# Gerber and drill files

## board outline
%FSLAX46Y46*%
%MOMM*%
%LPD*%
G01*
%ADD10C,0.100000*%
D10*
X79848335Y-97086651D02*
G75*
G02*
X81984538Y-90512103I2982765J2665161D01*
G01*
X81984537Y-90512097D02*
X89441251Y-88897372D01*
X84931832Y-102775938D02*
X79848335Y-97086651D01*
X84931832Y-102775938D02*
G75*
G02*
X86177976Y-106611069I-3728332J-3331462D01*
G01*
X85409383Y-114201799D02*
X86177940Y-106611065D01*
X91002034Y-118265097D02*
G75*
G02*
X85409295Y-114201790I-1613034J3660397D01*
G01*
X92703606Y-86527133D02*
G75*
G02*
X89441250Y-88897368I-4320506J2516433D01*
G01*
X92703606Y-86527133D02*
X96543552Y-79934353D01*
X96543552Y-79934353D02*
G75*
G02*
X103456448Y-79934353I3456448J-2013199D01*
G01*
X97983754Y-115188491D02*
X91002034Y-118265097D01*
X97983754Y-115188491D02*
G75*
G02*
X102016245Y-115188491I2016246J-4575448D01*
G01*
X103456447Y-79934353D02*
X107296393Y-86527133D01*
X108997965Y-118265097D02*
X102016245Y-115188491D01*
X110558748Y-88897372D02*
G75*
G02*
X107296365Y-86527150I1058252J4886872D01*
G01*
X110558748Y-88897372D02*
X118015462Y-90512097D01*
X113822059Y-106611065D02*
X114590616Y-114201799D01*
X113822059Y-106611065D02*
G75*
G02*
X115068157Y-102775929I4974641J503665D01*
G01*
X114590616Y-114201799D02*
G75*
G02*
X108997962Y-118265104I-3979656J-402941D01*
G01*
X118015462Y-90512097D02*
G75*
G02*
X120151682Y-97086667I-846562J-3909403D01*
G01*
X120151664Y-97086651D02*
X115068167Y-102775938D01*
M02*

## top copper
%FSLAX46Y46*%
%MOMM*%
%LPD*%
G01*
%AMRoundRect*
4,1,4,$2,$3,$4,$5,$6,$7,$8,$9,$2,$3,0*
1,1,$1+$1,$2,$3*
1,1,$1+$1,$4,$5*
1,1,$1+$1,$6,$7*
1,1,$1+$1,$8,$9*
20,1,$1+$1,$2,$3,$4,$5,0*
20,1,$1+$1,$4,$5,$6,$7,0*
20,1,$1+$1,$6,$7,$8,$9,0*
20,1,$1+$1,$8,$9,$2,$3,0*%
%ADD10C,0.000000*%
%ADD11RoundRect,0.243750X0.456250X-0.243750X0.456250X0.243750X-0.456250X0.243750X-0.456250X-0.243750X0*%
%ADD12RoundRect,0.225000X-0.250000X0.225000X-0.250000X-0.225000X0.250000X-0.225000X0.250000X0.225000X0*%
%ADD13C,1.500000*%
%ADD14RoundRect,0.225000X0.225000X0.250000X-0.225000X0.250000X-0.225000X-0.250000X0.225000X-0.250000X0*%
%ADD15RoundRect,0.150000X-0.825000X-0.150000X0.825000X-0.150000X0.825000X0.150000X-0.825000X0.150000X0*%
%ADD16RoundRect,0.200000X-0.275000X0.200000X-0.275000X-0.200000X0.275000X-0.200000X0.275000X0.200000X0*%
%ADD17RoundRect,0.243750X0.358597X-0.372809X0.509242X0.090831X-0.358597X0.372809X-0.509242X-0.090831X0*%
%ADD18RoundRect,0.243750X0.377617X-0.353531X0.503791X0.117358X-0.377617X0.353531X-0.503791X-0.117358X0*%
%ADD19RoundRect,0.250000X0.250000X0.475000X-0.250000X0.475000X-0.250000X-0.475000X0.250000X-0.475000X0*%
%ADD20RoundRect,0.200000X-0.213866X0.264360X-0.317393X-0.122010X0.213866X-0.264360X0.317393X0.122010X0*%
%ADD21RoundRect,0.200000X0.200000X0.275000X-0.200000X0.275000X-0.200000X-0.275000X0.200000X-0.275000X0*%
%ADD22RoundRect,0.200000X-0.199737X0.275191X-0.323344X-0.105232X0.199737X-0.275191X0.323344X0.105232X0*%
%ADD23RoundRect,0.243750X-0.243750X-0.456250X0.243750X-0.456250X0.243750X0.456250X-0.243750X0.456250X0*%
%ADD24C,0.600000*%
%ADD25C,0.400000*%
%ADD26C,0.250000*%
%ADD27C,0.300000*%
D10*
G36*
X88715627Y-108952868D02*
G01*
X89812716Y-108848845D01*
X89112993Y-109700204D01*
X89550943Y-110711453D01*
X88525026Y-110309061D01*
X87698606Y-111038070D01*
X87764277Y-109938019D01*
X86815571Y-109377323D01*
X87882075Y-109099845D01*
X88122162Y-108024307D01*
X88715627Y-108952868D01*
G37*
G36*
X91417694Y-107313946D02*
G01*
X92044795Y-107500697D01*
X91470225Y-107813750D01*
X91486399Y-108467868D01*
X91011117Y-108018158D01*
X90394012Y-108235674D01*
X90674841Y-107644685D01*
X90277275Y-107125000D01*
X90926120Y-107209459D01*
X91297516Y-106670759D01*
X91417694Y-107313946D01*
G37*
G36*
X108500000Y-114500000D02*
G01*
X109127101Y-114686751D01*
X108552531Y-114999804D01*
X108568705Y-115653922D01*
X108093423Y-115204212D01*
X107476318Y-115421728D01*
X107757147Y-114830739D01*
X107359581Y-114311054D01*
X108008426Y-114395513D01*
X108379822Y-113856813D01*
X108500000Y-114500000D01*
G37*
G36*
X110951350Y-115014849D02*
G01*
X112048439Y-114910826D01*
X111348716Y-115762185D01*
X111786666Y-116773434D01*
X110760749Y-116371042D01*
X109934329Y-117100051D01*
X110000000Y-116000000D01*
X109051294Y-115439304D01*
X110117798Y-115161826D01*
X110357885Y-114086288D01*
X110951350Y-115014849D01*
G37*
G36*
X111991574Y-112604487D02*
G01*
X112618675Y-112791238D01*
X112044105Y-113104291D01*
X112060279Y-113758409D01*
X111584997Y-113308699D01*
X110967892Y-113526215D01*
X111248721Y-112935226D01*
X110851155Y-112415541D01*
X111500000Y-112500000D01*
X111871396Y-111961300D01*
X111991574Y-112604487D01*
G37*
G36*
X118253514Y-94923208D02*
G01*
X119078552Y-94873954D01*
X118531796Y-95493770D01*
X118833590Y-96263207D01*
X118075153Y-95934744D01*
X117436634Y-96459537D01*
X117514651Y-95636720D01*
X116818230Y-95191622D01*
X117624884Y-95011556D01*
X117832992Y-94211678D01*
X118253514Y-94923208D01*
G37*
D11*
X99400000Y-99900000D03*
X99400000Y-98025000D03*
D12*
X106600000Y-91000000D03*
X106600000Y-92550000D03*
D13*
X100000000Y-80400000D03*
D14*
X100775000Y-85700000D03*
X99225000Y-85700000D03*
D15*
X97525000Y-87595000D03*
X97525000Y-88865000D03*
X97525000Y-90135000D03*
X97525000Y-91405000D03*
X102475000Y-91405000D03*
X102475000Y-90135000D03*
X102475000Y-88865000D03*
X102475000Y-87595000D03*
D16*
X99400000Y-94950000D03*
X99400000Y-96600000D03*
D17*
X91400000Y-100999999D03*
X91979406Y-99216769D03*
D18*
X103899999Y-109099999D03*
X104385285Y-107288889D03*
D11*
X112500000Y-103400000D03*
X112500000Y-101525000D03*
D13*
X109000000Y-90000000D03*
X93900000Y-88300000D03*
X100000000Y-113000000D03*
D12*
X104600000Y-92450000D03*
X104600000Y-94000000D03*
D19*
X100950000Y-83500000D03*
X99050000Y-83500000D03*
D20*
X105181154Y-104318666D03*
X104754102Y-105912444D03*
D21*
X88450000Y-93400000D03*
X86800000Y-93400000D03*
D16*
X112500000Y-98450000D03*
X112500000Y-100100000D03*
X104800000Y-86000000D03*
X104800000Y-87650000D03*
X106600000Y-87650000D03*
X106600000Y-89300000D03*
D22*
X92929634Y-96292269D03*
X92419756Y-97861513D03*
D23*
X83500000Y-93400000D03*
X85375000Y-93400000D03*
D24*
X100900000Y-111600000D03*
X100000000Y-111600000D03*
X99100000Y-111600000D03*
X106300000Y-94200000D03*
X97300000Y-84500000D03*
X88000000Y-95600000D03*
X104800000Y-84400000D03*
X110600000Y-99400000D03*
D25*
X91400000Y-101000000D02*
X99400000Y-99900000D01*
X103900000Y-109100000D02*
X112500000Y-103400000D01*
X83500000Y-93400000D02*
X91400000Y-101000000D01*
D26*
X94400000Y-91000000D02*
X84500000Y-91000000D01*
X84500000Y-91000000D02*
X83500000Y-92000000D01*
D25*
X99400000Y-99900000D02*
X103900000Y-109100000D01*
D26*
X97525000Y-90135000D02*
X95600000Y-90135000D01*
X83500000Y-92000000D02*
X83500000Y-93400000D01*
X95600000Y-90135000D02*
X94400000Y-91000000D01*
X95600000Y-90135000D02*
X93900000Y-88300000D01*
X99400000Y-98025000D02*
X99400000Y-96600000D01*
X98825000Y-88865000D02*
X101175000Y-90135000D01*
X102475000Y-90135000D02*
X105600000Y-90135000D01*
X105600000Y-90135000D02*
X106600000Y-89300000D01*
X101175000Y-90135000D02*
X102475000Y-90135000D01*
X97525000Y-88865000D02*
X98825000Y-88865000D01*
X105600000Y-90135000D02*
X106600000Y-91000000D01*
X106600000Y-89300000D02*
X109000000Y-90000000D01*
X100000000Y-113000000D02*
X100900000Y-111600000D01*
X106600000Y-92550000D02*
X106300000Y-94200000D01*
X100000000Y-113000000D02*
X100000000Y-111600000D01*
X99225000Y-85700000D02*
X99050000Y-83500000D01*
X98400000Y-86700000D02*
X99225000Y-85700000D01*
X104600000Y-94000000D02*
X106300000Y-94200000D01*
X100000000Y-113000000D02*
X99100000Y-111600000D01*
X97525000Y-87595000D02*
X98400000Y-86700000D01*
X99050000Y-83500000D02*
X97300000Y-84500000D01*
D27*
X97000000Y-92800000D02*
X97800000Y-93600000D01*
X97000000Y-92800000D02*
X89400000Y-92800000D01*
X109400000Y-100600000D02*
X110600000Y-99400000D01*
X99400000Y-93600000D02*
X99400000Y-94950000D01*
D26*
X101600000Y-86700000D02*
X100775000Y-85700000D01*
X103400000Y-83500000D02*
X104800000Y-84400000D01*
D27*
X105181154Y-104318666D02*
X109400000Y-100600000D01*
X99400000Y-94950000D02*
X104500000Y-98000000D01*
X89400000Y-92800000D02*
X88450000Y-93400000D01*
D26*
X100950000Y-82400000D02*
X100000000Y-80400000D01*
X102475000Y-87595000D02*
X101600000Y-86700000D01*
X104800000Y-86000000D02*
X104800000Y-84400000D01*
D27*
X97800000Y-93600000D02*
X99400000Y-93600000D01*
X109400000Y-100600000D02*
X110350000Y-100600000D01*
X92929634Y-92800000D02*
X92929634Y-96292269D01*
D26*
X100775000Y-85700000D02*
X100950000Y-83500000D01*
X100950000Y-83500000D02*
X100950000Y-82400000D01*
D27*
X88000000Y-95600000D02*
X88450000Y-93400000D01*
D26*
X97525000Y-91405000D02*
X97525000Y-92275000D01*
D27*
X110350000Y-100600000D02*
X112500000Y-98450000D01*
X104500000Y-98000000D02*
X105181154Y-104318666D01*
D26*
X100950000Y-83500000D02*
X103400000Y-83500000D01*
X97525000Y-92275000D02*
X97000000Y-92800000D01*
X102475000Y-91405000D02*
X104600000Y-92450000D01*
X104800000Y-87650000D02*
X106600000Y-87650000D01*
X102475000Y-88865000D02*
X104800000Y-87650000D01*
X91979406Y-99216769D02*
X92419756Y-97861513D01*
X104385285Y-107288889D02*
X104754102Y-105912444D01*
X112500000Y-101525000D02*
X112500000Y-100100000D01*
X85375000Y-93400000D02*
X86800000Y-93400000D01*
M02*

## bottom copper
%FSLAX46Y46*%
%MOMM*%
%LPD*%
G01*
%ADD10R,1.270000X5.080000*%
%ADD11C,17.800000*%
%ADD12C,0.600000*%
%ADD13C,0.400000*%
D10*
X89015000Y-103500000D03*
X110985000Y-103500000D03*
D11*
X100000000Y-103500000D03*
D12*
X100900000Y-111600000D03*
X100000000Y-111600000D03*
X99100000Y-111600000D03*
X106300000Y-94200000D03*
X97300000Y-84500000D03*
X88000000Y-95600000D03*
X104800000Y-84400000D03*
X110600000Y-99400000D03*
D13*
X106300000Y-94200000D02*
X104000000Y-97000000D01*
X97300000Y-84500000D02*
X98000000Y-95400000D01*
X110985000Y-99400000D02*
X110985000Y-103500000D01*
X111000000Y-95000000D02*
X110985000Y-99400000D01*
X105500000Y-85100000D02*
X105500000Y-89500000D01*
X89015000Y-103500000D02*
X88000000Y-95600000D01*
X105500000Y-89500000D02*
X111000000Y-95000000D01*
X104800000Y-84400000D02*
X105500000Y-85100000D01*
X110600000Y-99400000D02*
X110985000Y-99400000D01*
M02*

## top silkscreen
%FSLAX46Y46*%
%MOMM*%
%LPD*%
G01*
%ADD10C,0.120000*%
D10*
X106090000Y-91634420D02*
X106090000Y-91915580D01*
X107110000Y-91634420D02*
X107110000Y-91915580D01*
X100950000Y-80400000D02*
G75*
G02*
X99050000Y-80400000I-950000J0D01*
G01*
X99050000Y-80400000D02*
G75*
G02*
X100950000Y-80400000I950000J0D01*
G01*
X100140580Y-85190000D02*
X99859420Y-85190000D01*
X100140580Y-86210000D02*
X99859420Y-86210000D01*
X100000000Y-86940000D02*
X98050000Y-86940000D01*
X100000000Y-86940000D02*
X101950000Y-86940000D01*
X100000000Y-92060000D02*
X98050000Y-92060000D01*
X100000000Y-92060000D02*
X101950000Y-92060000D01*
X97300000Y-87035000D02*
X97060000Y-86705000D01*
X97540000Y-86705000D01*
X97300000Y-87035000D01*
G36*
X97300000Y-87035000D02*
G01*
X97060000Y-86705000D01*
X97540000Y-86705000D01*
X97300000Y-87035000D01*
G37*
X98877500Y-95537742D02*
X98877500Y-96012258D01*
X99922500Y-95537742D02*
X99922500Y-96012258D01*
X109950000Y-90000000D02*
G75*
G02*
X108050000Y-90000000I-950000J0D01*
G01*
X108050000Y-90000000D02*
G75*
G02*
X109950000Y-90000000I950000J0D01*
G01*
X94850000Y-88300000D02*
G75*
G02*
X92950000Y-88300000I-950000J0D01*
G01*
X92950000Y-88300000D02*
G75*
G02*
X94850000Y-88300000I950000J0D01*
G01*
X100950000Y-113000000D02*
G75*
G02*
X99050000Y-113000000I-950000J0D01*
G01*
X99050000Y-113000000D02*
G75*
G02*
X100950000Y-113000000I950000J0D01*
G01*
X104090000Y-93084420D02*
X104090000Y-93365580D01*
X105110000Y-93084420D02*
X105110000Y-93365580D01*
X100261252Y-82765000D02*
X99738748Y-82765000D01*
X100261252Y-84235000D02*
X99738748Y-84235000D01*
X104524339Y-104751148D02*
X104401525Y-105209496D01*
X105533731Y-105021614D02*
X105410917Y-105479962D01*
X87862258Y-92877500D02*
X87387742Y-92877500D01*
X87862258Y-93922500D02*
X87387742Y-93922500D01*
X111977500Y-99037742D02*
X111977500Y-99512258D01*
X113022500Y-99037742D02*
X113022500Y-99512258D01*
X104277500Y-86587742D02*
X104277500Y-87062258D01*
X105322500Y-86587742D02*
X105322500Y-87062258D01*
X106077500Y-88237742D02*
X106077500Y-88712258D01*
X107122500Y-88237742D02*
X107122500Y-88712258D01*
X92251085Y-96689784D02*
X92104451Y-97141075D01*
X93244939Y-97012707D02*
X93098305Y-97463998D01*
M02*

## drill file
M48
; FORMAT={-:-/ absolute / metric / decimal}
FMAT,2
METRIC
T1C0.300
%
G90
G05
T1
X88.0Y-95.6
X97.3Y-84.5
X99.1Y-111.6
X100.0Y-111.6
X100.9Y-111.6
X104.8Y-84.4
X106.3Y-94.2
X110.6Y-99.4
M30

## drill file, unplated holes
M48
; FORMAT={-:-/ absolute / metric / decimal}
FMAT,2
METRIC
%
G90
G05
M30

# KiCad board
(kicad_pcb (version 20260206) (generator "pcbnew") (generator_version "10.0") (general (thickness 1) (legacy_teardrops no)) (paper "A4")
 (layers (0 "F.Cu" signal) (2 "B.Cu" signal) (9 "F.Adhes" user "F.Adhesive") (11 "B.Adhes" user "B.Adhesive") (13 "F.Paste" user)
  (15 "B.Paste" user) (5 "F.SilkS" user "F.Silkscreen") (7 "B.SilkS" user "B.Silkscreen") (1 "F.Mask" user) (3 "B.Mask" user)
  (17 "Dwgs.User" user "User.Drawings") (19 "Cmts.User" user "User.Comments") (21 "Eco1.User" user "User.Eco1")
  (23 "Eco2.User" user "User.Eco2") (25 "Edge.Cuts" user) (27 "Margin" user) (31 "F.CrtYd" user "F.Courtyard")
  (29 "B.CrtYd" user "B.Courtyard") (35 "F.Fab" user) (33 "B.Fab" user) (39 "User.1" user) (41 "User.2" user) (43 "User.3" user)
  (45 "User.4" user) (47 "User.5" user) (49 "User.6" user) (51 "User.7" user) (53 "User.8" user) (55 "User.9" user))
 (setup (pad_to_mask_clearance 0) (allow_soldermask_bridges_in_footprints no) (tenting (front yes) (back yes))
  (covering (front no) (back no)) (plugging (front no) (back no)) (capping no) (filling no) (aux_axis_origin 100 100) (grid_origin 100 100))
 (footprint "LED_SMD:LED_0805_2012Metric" (layer "F.Cu") (at 99.4 98.9625 90)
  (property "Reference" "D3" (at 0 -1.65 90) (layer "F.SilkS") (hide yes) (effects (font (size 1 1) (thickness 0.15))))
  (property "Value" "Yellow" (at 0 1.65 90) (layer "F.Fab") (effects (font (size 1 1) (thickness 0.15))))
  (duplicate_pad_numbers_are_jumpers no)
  (pad "1" smd roundrect (at -0.9375 0 90) (size 0.975 1.4) (layers "F.Cu" "F.Mask" "F.Paste") (roundrect_rratio 0.25) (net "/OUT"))
  (pad "2" smd roundrect (at 0.9375 0 90) (size 0.975 1.4) (layers "F.Cu" "F.Mask" "F.Paste") (roundrect_rratio 0.25) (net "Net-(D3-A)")))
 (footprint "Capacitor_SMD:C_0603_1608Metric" (layer "F.Cu") (at 106.6 91.775 -90)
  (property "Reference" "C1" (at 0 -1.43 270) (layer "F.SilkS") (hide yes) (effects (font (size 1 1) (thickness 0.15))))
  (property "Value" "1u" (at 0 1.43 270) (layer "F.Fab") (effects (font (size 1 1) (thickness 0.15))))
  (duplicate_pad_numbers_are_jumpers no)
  (fp_line (start -0.14058 0.51) (end 0.14058 0.51) (stroke (width 0.12) (type solid)) (layer "F.SilkS"))
  (fp_line (start -0.14058 -0.51) (end 0.14058 -0.51) (stroke (width 0.12) (type solid)) (layer "F.SilkS"))
  (pad "1" smd roundrect (at -0.775 0 270) (size 0.9 0.95) (layers "F.Cu" "F.Mask" "F.Paste") (roundrect_rratio 0.25) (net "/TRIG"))
  (pad "2" smd roundrect (at 0.775 0 270) (size 0.9 0.95) (layers "F.Cu" "F.Mask" "F.Paste") (roundrect_rratio 0.25) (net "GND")))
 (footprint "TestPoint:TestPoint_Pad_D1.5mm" (layer "F.Cu") (at 100 80.4)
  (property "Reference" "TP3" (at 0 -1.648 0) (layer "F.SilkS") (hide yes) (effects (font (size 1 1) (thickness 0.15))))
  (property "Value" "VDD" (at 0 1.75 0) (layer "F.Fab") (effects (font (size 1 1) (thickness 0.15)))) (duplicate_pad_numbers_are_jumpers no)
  (fp_circle (center 0 0) (end 0 0.95) (stroke (width 0.12) (type solid)) (fill no) (layer "F.SilkS"))
  (pad "1" smd circle (at 0 0) (size 1.5 1.5) (layers "F.Cu" "F.Mask") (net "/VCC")))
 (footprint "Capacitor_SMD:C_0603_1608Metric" (layer "F.Cu") (at 100 85.7 180)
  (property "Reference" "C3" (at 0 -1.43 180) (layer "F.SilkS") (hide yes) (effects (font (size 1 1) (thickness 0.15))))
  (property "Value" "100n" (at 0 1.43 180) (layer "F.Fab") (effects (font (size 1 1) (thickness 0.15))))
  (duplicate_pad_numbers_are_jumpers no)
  (fp_line (start -0.14058 0.51) (end 0.14058 0.51) (stroke (width 0.12) (type solid)) (layer "F.SilkS"))
  (fp_line (start -0.14058 -0.51) (end 0.14058 -0.51) (stroke (width 0.12) (type solid)) (layer "F.SilkS"))
  (pad "1" smd roundrect (at -0.775 0 180) (size 0.9 0.95) (layers "F.Cu" "F.Mask" "F.Paste") (roundrect_rratio 0.25) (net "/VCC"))
  (pad "2" smd roundrect (at 0.775 0 180) (size 0.9 0.95) (layers "F.Cu" "F.Mask" "F.Paste") (roundrect_rratio 0.25) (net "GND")))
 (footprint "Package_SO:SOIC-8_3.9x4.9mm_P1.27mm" (layer "F.Cu") (at 100 89.5)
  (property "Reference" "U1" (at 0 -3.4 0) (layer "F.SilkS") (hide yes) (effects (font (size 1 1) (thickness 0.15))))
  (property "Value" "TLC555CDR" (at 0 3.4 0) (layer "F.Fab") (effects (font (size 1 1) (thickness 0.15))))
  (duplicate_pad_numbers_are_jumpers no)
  (fp_line (start 0 -2.56) (end -1.95 -2.56) (stroke (width 0.12) (type solid)) (layer "F.SilkS"))
  (fp_line (start 0 -2.56) (end 1.95 -2.56) (stroke (width 0.12) (type solid)) (layer "F.SilkS"))
  (fp_line (start 0 2.56) (end -1.95 2.56) (stroke (width 0.12) (type solid)) (layer "F.SilkS"))
  (fp_line (start 0 2.56) (end 1.95 2.56) (stroke (width 0.12) (type solid)) (layer "F.SilkS"))
  (fp_poly
   (pts (xy -2.7 -2.465) (xy -2.94 -2.795) (xy -2.46 -2.795) (xy -2.7 -2.465)) (stroke (width 0.12) (type solid)) (fill yes)
   (layer "F.SilkS"))
  (pad "1" smd roundrect (at -2.475 -1.905) (size 1.95 0.6) (layers "F.Cu" "F.Mask" "F.Paste") (roundrect_rratio 0.25) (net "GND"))
  (pad "2" smd roundrect (at -2.475 -0.635) (size 1.95 0.6) (layers "F.Cu" "F.Mask" "F.Paste") (roundrect_rratio 0.25) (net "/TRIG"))
  (pad "3" smd roundrect (at -2.475 0.635) (size 1.95 0.6) (layers "F.Cu" "F.Mask" "F.Paste") (roundrect_rratio 0.25) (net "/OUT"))
  (pad "4" smd roundrect (at -2.475 1.905) (size 1.95 0.6) (layers "F.Cu" "F.Mask" "F.Paste") (roundrect_rratio 0.25) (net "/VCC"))
  (pad "5" smd roundrect (at 2.475 1.905) (size 1.95 0.6) (layers "F.Cu" "F.Mask" "F.Paste") (roundrect_rratio 0.25) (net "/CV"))
  (pad "6" smd roundrect (at 2.475 0.635) (size 1.95 0.6) (layers "F.Cu" "F.Mask" "F.Paste") (roundrect_rratio 0.25) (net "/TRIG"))
  (pad "7" smd roundrect (at 2.475 -0.635) (size 1.95 0.6) (layers "F.Cu" "F.Mask" "F.Paste") (roundrect_rratio 0.25) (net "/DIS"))
  (pad "8" smd roundrect (at 2.475 -1.905) (size 1.95 0.6) (layers "F.Cu" "F.Mask" "F.Paste") (roundrect_rratio 0.25) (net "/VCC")))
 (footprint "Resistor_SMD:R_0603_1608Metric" (layer "F.Cu") (at 99.4 95.775 -90)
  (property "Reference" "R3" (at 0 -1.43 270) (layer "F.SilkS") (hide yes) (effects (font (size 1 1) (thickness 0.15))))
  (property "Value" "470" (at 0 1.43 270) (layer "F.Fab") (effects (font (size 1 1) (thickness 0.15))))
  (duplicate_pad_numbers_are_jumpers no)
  (fp_line (start -0.237258 0.5225) (end 0.237258 0.5225) (stroke (width 0.12) (type solid)) (layer "F.SilkS"))
  (fp_line (start -0.237258 -0.5225) (end 0.237258 -0.5225) (stroke (width 0.12) (type solid)) (layer "F.SilkS"))
  (pad "1" smd roundrect (at -0.825 0 270) (size 0.8 0.95) (layers "F.Cu" "F.Mask" "F.Paste") (roundrect_rratio 0.25) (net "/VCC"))
  (pad "2" smd roundrect (at 0.825 0 270) (size 0.8 0.95) (layers "F.Cu" "F.Mask" "F.Paste") (roundrect_rratio 0.25) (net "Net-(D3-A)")))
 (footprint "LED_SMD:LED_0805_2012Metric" (layer "F.Cu") (at 91.689703 100.108384 72)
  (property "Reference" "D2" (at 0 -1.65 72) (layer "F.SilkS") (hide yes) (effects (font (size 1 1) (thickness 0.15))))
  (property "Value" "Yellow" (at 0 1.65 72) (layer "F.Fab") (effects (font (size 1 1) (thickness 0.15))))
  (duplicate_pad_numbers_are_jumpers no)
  (pad "1" smd roundrect (at -0.937499 0 72) (size 0.975 1.4) (layers "F.Cu" "F.Mask" "F.Paste") (roundrect_rratio 0.25) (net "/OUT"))
  (pad "2" smd roundrect (at 0.937499 0 72) (size 0.975 1.4) (layers "F.Cu" "F.Mask" "F.Paste") (roundrect_rratio 0.25) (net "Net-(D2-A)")))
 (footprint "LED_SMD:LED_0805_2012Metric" (layer "F.Cu") (at 104.142642 108.194444 75)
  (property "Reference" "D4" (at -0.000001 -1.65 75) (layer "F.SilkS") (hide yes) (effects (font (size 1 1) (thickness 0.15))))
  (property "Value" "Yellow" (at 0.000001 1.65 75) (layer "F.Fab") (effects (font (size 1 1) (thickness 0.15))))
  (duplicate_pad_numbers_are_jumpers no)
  (pad "1" smd roundrect (at -0.9375 0 75) (size 0.975 1.4) (layers "F.Cu" "F.Mask" "F.Paste") (roundrect_rratio 0.25) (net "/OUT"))
  (pad "2" smd roundrect (at 0.9375 0 75) (size 0.975 1.4) (layers "F.Cu" "F.Mask" "F.Paste") (roundrect_rratio 0.25) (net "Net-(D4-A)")))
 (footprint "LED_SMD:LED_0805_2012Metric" (layer "F.Cu") (at 112.5 102.4625 90)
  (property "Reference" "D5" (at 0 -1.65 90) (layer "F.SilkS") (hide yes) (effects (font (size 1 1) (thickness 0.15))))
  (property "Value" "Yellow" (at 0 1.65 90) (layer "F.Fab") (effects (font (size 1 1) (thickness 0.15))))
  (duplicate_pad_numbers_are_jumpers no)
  (pad "1" smd roundrect (at -0.9375 0 90) (size 0.975 1.4) (layers "F.Cu" "F.Mask" "F.Paste") (roundrect_rratio 0.25) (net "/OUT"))
  (pad "2" smd roundrect (at 0.9375 0 90) (size 0.975 1.4) (layers "F.Cu" "F.Mask" "F.Paste") (roundrect_rratio 0.25) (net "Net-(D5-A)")))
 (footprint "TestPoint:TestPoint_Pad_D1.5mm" (layer "F.Cu") (at 109 90)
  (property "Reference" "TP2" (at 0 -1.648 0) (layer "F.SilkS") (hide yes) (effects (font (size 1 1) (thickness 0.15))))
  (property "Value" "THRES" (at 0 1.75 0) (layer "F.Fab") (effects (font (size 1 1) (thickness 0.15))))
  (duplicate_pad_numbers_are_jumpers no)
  (fp_circle (center 0 0) (end 0 0.95) (stroke (width 0.12) (type solid)) (fill no) (layer "F.SilkS"))
  (pad "1" smd circle (at 0 0) (size 1.5 1.5) (layers "F.Cu" "F.Mask") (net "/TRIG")))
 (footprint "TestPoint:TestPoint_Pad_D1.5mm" (layer "F.Cu") (at 93.9 88.3)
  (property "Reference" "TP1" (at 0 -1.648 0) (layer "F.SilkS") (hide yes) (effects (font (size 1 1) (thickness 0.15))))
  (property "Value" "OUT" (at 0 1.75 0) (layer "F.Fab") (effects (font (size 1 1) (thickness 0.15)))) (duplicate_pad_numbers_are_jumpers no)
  (fp_circle (center 0 0) (end 0 0.95) (stroke (width 0.12) (type solid)) (fill no) (layer "F.SilkS"))
  (pad "1" smd circle (at 0 0) (size 1.5 1.5) (layers "F.Cu" "F.Mask") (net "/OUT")))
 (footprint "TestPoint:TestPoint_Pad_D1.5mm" (layer "F.Cu") (at 100 113)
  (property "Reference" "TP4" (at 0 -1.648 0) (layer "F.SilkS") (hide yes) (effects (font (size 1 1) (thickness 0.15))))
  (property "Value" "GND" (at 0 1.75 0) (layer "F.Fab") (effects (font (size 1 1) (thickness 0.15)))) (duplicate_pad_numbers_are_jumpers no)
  (fp_circle (center 0 0) (end 0 0.95) (stroke (width 0.12) (type solid)) (fill no) (layer "F.SilkS"))
  (pad "1" smd circle (at 0 0) (size 1.5 1.5) (layers "F.Cu" "F.Mask") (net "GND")))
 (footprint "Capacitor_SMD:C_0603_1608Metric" (layer "F.Cu") (at 104.6 93.225 -90)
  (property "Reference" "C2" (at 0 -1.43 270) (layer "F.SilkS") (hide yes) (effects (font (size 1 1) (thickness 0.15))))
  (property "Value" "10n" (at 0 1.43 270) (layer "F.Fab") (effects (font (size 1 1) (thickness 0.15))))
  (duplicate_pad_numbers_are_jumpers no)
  (fp_line (start -0.14058 0.51) (end 0.14058 0.51) (stroke (width 0.12) (type solid)) (layer "F.SilkS"))
  (fp_line (start -0.14058 -0.51) (end 0.14058 -0.51) (stroke (width 0.12) (type solid)) (layer "F.SilkS"))
  (pad "1" smd roundrect (at -0.775 0 270) (size 0.9 0.95) (layers "F.Cu" "F.Mask" "F.Paste") (roundrect_rratio 0.25) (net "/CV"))
  (pad "2" smd roundrect (at 0.775 0 270) (size 0.9 0.95) (layers "F.Cu" "F.Mask" "F.Paste") (roundrect_rratio 0.25) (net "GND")))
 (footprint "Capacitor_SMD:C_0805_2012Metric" (layer "F.Cu") (at 100 83.5 180)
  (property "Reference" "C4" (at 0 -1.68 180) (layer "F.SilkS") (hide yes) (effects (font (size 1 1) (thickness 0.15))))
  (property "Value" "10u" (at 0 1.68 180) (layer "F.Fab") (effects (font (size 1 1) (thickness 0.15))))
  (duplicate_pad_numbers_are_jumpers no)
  (fp_line (start -0.261252 0.735) (end 0.261252 0.735) (stroke (width 0.12) (type solid)) (layer "F.SilkS"))
  (fp_line (start -0.261252 -0.735) (end 0.261252 -0.735) (stroke (width 0.12) (type solid)) (layer "F.SilkS"))
  (pad "1" smd roundrect (at -0.95 0 180) (size 1 1.45) (layers "F.Cu" "F.Mask" "F.Paste") (roundrect_rratio 0.25) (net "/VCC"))
  (pad "2" smd roundrect (at 0.95 0 180) (size 1 1.45) (layers "F.Cu" "F.Mask" "F.Paste") (roundrect_rratio 0.25) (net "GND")))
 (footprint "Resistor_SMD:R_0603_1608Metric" (layer "F.Cu") (at 104.967628 105.115555 -105)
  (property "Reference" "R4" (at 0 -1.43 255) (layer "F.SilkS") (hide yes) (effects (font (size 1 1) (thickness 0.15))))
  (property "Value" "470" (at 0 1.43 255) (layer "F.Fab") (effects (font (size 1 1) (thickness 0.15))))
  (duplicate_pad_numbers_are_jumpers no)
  (fp_line (start -0.237258 0.5225) (end 0.237258 0.5225) (stroke (width 0.12) (type solid)) (layer "F.SilkS"))
  (fp_line (start -0.237258 -0.5225) (end 0.237258 -0.5225) (stroke (width 0.12) (type solid)) (layer "F.SilkS"))
  (pad "1" smd roundrect (at -0.825 0 255) (size 0.8 0.95) (layers "F.Cu" "F.Mask" "F.Paste") (roundrect_rratio 0.25) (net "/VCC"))
  (pad "2" smd roundrect (at 0.825 0 255) (size 0.8 0.95) (layers "F.Cu" "F.Mask" "F.Paste") (roundrect_rratio 0.25) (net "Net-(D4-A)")))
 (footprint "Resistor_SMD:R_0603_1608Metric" (layer "F.Cu") (at 87.625 93.4 180)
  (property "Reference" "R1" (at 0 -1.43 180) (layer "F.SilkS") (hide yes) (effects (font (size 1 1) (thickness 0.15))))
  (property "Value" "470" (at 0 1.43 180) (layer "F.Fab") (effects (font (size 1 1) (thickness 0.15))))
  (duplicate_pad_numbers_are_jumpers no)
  (fp_line (start -0.237258 0.5225) (end 0.237258 0.5225) (stroke (width 0.12) (type solid)) (layer "F.SilkS"))
  (fp_line (start -0.237258 -0.5225) (end 0.237258 -0.5225) (stroke (width 0.12) (type solid)) (layer "F.SilkS"))
  (pad "1" smd roundrect (at -0.825 0 180) (size 0.8 0.95) (layers "F.Cu" "F.Mask" "F.Paste") (roundrect_rratio 0.25) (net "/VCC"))
  (pad "2" smd roundrect (at 0.825 0 180) (size 0.8 0.95) (layers "F.Cu" "F.Mask" "F.Paste") (roundrect_rratio 0.25) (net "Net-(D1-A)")))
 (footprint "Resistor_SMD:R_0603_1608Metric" (layer "F.Cu") (at 112.5 99.275 -90)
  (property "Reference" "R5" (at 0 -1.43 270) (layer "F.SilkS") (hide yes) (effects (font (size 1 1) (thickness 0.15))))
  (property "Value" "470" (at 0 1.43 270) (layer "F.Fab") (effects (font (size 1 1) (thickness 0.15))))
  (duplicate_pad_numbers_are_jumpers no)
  (fp_line (start -0.237258 0.5225) (end 0.237258 0.5225) (stroke (width 0.12) (type solid)) (layer "F.SilkS"))
  (fp_line (start -0.237258 -0.5225) (end 0.237258 -0.5225) (stroke (width 0.12) (type solid)) (layer "F.SilkS"))
  (pad "1" smd roundrect (at -0.825 0 270) (size 0.8 0.95) (layers "F.Cu" "F.Mask" "F.Paste") (roundrect_rratio 0.25) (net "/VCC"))
  (pad "2" smd roundrect (at 0.825 0 270) (size 0.8 0.95) (layers "F.Cu" "F.Mask" "F.Paste") (roundrect_rratio 0.25) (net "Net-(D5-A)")))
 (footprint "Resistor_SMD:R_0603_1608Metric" (layer "F.Cu") (at 104.8 86.825 -90)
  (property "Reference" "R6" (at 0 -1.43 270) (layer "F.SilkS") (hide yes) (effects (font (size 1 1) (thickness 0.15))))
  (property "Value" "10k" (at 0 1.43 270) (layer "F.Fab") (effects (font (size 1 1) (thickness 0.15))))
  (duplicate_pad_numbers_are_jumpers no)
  (fp_line (start -0.237258 0.5225) (end 0.237258 0.5225) (stroke (width 0.12) (type solid)) (layer "F.SilkS"))
  (fp_line (start -0.237258 -0.5225) (end 0.237258 -0.5225) (stroke (width 0.12) (type solid)) (layer "F.SilkS"))
  (pad "1" smd roundrect (at -0.825 0 270) (size 0.8 0.95) (layers "F.Cu" "F.Mask" "F.Paste") (roundrect_rratio 0.25) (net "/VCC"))
  (pad "2" smd roundrect (at 0.825 0 270) (size 0.8 0.95) (layers "F.Cu" "F.Mask" "F.Paste") (roundrect_rratio 0.25) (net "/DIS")))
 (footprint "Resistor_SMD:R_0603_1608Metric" (layer "F.Cu") (at 106.6 88.475 -90)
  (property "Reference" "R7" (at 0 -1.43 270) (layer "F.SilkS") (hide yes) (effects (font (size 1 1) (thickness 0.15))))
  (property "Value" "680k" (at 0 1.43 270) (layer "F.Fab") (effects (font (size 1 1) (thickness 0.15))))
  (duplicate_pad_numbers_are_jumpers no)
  (fp_line (start -0.237258 0.5225) (end 0.237258 0.5225) (stroke (width 0.12) (type solid)) (layer "F.SilkS"))
  (fp_line (start -0.237258 -0.5225) (end 0.237258 -0.5225) (stroke (width 0.12) (type solid)) (layer "F.SilkS"))
  (pad "1" smd roundrect (at -0.825 0 270) (size 0.8 0.95) (layers "F.Cu" "F.Mask" "F.Paste") (roundrect_rratio 0.25) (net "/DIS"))
  (pad "2" smd roundrect (at 0.825 0 270) (size 0.8 0.95) (layers "F.Cu" "F.Mask" "F.Paste") (roundrect_rratio 0.25) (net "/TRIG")))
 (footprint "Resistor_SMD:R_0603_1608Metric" (layer "F.Cu") (at 92.674695 97.076891 -108)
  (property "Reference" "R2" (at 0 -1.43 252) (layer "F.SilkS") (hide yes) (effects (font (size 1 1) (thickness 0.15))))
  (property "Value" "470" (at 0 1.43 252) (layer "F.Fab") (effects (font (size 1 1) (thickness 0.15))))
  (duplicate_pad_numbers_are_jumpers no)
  (fp_line (start -0.237258 0.5225) (end 0.237258 0.5225) (stroke (width 0.12) (type solid)) (layer "F.SilkS"))
  (fp_line (start -0.237258 -0.5225) (end 0.237258 -0.5225) (stroke (width 0.12) (type solid)) (layer "F.SilkS"))
  (pad "1" smd roundrect (at -0.825 0 252) (size 0.8 0.95) (layers "F.Cu" "F.Mask" "F.Paste") (roundrect_rratio 0.25) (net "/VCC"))
  (pad "2" smd roundrect (at 0.825 0 252) (size 0.8 0.95) (layers "F.Cu" "F.Mask" "F.Paste") (roundrect_rratio 0.25) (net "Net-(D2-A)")))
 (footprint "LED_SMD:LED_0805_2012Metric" (layer "F.Cu") (at 84.4375 93.4)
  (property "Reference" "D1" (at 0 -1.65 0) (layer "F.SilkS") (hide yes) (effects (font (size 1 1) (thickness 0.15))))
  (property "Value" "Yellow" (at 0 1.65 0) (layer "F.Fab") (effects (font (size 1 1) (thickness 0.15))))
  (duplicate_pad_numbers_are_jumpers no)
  (pad "1" smd roundrect (at -0.9375 0) (size 0.975 1.4) (layers "F.Cu" "F.Mask" "F.Paste") (roundrect_rratio 0.25) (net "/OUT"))
  (pad "2" smd roundrect (at 0.9375 0) (size 0.975 1.4) (layers "F.Cu" "F.Mask" "F.Paste") (roundrect_rratio 0.25) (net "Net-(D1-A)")))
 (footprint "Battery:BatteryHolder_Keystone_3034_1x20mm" (layer "B.Cu") (at 100 103.5)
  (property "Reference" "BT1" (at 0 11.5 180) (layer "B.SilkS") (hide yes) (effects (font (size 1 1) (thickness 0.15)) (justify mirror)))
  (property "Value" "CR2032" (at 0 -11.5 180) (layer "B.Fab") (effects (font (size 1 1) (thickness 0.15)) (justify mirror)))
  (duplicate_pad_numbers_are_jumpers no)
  (pad "1" smd rect (at -10.985 0) (size 1.27 5.08) (layers "B.Cu" "B.Mask" "B.Paste") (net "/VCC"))
  (pad "1" smd rect (at 10.985 0) (size 1.27 5.08) (layers "B.Cu" "B.Mask" "B.Paste") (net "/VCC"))
  (pad "2" smd circle (at 0 0) (size 17.8 17.8) (layers "B.Cu" "B.Mask") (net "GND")))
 (gr_poly
  (pts (xy 88.122162 108.024307) (xy 88.715627 108.952868) (xy 89.812716 108.848845) (xy 89.112993 109.700204) (xy 89.550943 110.711453)
   (xy 88.525026 110.309061) (xy 87.698606 111.03807) (xy 87.764277 109.938019) (xy 86.815571 109.377323) (xy 87.882075 109.099845))
  (stroke (width 0) (type default)) (fill yes) (layer "F.Cu"))
 (gr_poly
  (pts (xy 91.297516 106.670759) (xy 91.417694 107.313946) (xy 92.044795 107.500697) (xy 91.470225 107.81375) (xy 91.486399 108.467868)
   (xy 91.011117 108.018158) (xy 90.394012 108.235674) (xy 90.674841 107.644685) (xy 90.277275 107.125) (xy 90.92612 107.209459))
  (stroke (width 0) (type default)) (fill yes) (layer "F.Cu"))
 (gr_poly
  (pts (xy 108.379822 113.856813) (xy 108.5 114.5) (xy 109.127101 114.686751) (xy 108.552531 114.999804) (xy 108.568705 115.653922)
   (xy 108.093423 115.204212) (xy 107.476318 115.421728) (xy 107.757147 114.830739) (xy 107.359581 114.311054) (xy 108.008426 114.395513))
  (stroke (width 0) (type default)) (fill yes) (layer "F.Cu"))
 (gr_poly
  (pts (xy 110.357885 114.086288) (xy 110.95135 115.014849) (xy 112.048439 114.910826) (xy 111.348716 115.762185) (xy 111.786666 116.773434)
   (xy 110.760749 116.371042) (xy 109.934329 117.100051) (xy 110 116) (xy 109.051294 115.439304) (xy 110.117798 115.161826))
  (stroke (width 0) (type default)) (fill yes) (layer "F.Cu"))
 (gr_poly
  (pts (xy 111.871396 111.9613) (xy 111.991574 112.604487) (xy 112.618675 112.791238) (xy 112.044105 113.104291) (xy 112.060279 113.758409)
   (xy 111.584997 113.308699) (xy 110.967892 113.526215) (xy 111.248721 112.935226) (xy 110.851155 112.415541) (xy 111.5 112.5))
  (stroke (width 0) (type default)) (fill yes) (layer "F.Cu"))
 (gr_poly
  (pts (xy 117.832992 94.211678) (xy 118.253514 94.923208) (xy 119.078552 94.873954) (xy 118.531796 95.49377) (xy 118.83359 96.263207)
   (xy 118.075153 95.934744) (xy 117.436634 96.459537) (xy 117.514651 95.63672) (xy 116.81823 95.191622) (xy 117.624884 95.011556))
  (stroke (width 0) (type default)) (fill yes) (layer "F.Cu"))
 (gr_arc (start 79.848335 97.086651) (mid 79.026875 93.185418) (end 81.984537 90.512097) (stroke (width 0.1) (type default))
  (layer "Edge.Cuts"))
 (gr_line (start 81.984537 90.512097) (end 89.441251 88.897372) (stroke (width 0.1) (type default)) (layer "Edge.Cuts"))
 (gr_line (start 84.931832 102.775938) (end 79.848335 97.086651) (stroke (width 0.1) (type default)) (layer "Edge.Cuts"))
 (gr_arc (start 84.931832 102.775938) (mid 85.958664 104.562307) (end 86.17794 106.611065) (stroke (width 0.1) (type default))
  (layer "Edge.Cuts"))
 (gr_line (start 85.409383 114.201799) (end 86.17794 106.611065) (stroke (width 0.1) (type default)) (layer "Edge.Cuts"))
 (gr_arc (start 91.002034 118.265097) (mid 87.037896 117.840805) (end 85.409383 114.201799) (stroke (width 0.1) (type default))
  (layer "Edge.Cuts"))
 (gr_arc (start 92.703606 86.527133) (mid 91.321972 88.055723) (end 89.441251 88.897372) (stroke (width 0.1) (type default))
  (layer "Edge.Cuts"))
 (gr_line (start 92.703606 86.527133) (end 96.543552 79.934353) (stroke (width 0.1) (type default)) (layer "Edge.Cuts"))
 (gr_arc (start 96.543552 79.934353) (mid 100 77.947552) (end 103.456447 79.934353) (stroke (width 0.1) (type default)) (layer "Edge.Cuts"))
 (gr_line (start 97.983754 115.188491) (end 91.002034 118.265097) (stroke (width 0.1) (type default)) (layer "Edge.Cuts"))
 (gr_arc (start 97.983754 115.188491) (mid 100 114.763942) (end 102.016245 115.188491) (stroke (width 0.1) (type default))
  (layer "Edge.Cuts"))
 (gr_line (start 103.456447 79.934353) (end 107.296393 86.527133) (stroke (width 0.1) (type default)) (layer "Edge.Cuts"))
 (gr_line (start 108.997965 118.265097) (end 102.016245 115.188491) (stroke (width 0.1) (type default)) (layer "Edge.Cuts"))
 (gr_arc (start 110.558748 88.897372) (mid 108.678035 88.055711) (end 107.296393 86.527133) (stroke (width 0.1) (type default))
  (layer "Edge.Cuts"))
 (gr_line (start 110.558748 88.897372) (end 118.015462 90.512097) (stroke (width 0.1) (type default)) (layer "Edge.Cuts"))
 (gr_line (start 113.822059 106.611065) (end 114.590616 114.201799) (stroke (width 0.1) (type default)) (layer "Edge.Cuts"))
 (gr_arc (start 113.822059 106.611065) (mid 114.041346 104.562311) (end 115.068167 102.775938) (stroke (width 0.1) (type default))
  (layer "Edge.Cuts"))
 (gr_arc (start 114.590616 114.201799) (mid 112.962103 117.840805) (end 108.997965 118.265097) (stroke (width 0.1) (type default))
  (layer "Edge.Cuts"))
 (gr_arc (start 118.015462 90.512097) (mid 120.973124 93.185418) (end 120.151664 97.086651) (stroke (width 0.1) (type default))
  (layer "Edge.Cuts"))
 (gr_line (start 120.151664 97.086651) (end 115.068167 102.775938) (stroke (width 0.1) (type default)) (layer "Edge.Cuts"))
 (segment (start 91.4 101) (end 99.4 99.9) (width 0.4) (layer "F.Cu") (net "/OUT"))
 (segment (start 103.9 109.1) (end 112.5 103.4) (width 0.4) (layer "F.Cu") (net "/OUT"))
 (segment (start 83.5 93.4) (end 91.4 101) (width 0.4) (layer "F.Cu") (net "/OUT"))
 (segment (start 94.4 91) (end 84.5 91) (width 0.25) (layer "F.Cu") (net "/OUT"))
 (segment (start 84.5 91) (end 83.5 92) (width 0.25) (layer "F.Cu") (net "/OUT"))
 (segment (start 99.4 99.9) (end 103.9 109.1) (width 0.4) (layer "F.Cu") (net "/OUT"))
 (segment (start 97.525 90.135) (end 95.6 90.135) (width 0.25) (layer "F.Cu") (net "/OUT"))
 (segment (start 83.5 92) (end 83.5 93.4) (width 0.25) (layer "F.Cu") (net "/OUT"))
 (segment (start 95.6 90.135) (end 94.4 91) (width 0.25) (layer "F.Cu") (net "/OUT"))
 (segment (start 95.6 90.135) (end 93.9 88.3) (width 0.25) (layer "F.Cu") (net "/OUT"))
 (segment (start 99.4 98.025) (end 99.4 96.6) (width 0.25) (layer "F.Cu") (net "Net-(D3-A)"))
 (segment (start 98.825 88.865) (end 101.175 90.135) (width 0.25) (layer "F.Cu") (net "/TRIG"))
 (segment (start 102.475 90.135) (end 105.6 90.135) (width 0.25) (layer "F.Cu") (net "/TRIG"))
 (segment (start 105.6 90.135) (end 106.6 89.3) (width 0.25) (layer "F.Cu") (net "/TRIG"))
 (segment (start 101.175 90.135) (end 102.475 90.135) (width 0.25) (layer "F.Cu") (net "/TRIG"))
 (segment (start 97.525 88.865) (end 98.825 88.865) (width 0.25) (layer "F.Cu") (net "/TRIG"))
 (segment (start 105.6 90.135) (end 106.6 91) (width 0.25) (layer "F.Cu") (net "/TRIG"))
 (segment (start 106.6 89.3) (end 109 90) (width 0.25) (layer "F.Cu") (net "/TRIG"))
 (segment (start 100 113) (end 100.9 111.6) (width 0.25) (layer "F.Cu") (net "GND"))
 (segment (start 106.6 92.55) (end 106.3 94.2) (width 0.25) (layer "F.Cu") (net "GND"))
 (segment (start 100 113) (end 100 111.6) (width 0.25) (layer "F.Cu") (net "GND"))
 (segment (start 99.225 85.7) (end 99.05 83.5) (width 0.25) (layer "F.Cu") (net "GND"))
 (segment (start 98.4 86.7) (end 99.225 85.7) (width 0.25) (layer "F.Cu") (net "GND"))
 (segment (start 104.6 94) (end 106.3 94.2) (width 0.25) (layer "F.Cu") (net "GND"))
 (segment (start 100 113) (end 99.1 111.6) (width 0.25) (layer "F.Cu") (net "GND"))
 (segment (start 97.525 87.595) (end 98.4 86.7) (width 0.25) (layer "F.Cu") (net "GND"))
 (segment (start 99.05 83.5) (end 97.3 84.5) (width 0.25) (layer "F.Cu") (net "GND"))
 (via (at 100.9 111.6) (size 0.6) (drill 0.3) (layers "F.Cu" "B.Cu") (capping no) (covering (front no) (back no))
  (plugging (front no) (back no)) (filling no) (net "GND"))
 (via (at 100 111.6) (size 0.6) (drill 0.3) (layers "F.Cu" "B.Cu") (capping no) (covering (front no) (back no))
  (plugging (front no) (back no)) (filling no) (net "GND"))
 (via (at 99.1 111.6) (size 0.6) (drill 0.3) (layers "F.Cu" "B.Cu") (capping no) (covering (front no) (back no))
  (plugging (front no) (back no)) (filling no) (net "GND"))
 (via (at 106.3 94.2) (size 0.6) (drill 0.3) (layers "F.Cu" "B.Cu") (capping no) (covering (front no) (back no))
  (plugging (front no) (back no)) (filling no) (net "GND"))
 (via (at 97.3 84.5) (size 0.6) (drill 0.3) (layers "F.Cu" "B.Cu") (capping no) (covering (front no) (back no))
  (plugging (front no) (back no)) (filling no) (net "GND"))
 (segment (start 106.3 94.2) (end 104 97) (width 0.4) (layer "B.Cu") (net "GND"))
 (segment (start 97.3 84.5) (end 98 95.4) (width 0.4) (layer "B.Cu") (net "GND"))
 (segment (start 97 92.8) (end 97.8 93.6) (width 0.3) (layer "F.Cu") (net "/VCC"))
 (segment (start 97 92.8) (end 89.4 92.8) (width 0.3) (layer "F.Cu") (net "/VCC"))
 (segment (start 109.4 100.6) (end 110.6 99.4) (width 0.3) (layer "F.Cu") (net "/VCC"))
 (segment (start 99.4 93.6) (end 99.4 94.95) (width 0.3) (layer "F.Cu") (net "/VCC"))
 (segment (start 101.6 86.7) (end 100.775 85.7) (width 0.25) (layer "F.Cu") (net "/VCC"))
 (segment (start 103.4 83.5) (end 104.8 84.4) (width 0.25) (layer "F.Cu") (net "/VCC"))
 (segment (start 105.181154 104.318666) (end 109.4 100.6) (width 0.3) (layer "F.Cu") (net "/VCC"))
 (segment (start 99.4 94.95) (end 104.5 98) (width 0.3) (layer "F.Cu") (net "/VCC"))
 (segment (start 89.4 92.8) (end 88.45 93.4) (width 0.3) (layer "F.Cu") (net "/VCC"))
 (segment (start 100.95 82.4) (end 100 80.4) (width 0.25) (layer "F.Cu") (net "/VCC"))
 (segment (start 102.475 87.595) (end 101.6 86.7) (width 0.25) (layer "F.Cu") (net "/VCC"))
 (segment (start 104.8 86) (end 104.8 84.4) (width 0.25) (layer "F.Cu") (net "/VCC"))
 (segment (start 97.8 93.6) (end 99.4 93.6) (width 0.3) (layer "F.Cu") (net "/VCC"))
 (segment (start 109.4 100.6) (end 110.35 100.6) (width 0.3) (layer "F.Cu") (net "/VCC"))
 (segment (start 92.929634 92.8) (end 92.929634 96.292269) (width 0.3) (layer "F.Cu") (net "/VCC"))
 (segment (start 100.775 85.7) (end 100.95 83.5) (width 0.25) (layer "F.Cu") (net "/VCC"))
 (segment (start 100.95 83.5) (end 100.95 82.4) (width 0.25) (layer "F.Cu") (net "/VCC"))
 (segment (start 88 95.6) (end 88.45 93.4) (width 0.3) (layer "F.Cu") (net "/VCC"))
 (segment (start 97.525 91.405) (end 97.525 92.275) (width 0.25) (layer "F.Cu") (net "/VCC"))
 (segment (start 110.35 100.6) (end 112.5 98.45) (width 0.3) (layer "F.Cu") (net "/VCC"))
 (segment (start 104.5 98) (end 105.181154 104.318666) (width 0.3) (layer "F.Cu") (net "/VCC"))
 (segment (start 100.95 83.5) (end 103.4 83.5) (width 0.25) (layer "F.Cu") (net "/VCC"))
 (segment (start 97.525 92.275) (end 97 92.8) (width 0.25) (layer "F.Cu") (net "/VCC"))
 (via (at 88 95.6) (size 0.6) (drill 0.3) (layers "F.Cu" "B.Cu") (capping no) (covering (front no) (back no))
  (plugging (front no) (back no)) (filling no) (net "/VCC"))
 (via (at 104.8 84.4) (size 0.6) (drill 0.3) (layers "F.Cu" "B.Cu") (capping no) (covering (front no) (back no))
  (plugging (front no) (back no)) (filling no) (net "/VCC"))
 (via (at 110.6 99.4) (size 0.6) (drill 0.3) (layers "F.Cu" "B.Cu") (capping no) (covering (front no) (back no))
  (plugging (front no) (back no)) (filling no) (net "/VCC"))
 (segment (start 110.985 99.4) (end 110.985 103.5) (width 0.4) (layer "B.Cu") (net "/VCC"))
 (segment (start 111 95) (end 110.985 99.4) (width 0.4) (layer "B.Cu") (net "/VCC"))
 (segment (start 105.5 85.1) (end 105.5 89.5) (width 0.4) (layer "B.Cu") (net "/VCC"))
 (segment (start 89.015 103.5) (end 88 95.6) (width 0.4) (layer "B.Cu") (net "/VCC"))
 (segment (start 105.5 89.5) (end 111 95) (width 0.4) (layer "B.Cu") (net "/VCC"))
 (segment (start 104.8 84.4) (end 105.5 85.1) (width 0.4) (layer "B.Cu") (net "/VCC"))
 (segment (start 110.6 99.4) (end 110.985 99.4) (width 0.4) (layer "B.Cu") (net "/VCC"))
 (segment (start 102.475 91.405) (end 104.6 92.45) (width 0.25) (layer "F.Cu") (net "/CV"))
 (segment (start 104.8 87.65) (end 106.6 87.65) (width 0.25) (layer "F.Cu") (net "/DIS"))
 (segment (start 102.475 88.865) (end 104.8 87.65) (width 0.25) (layer "F.Cu") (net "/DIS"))
 (segment (start 91.979406 99.216769) (end 92.419756 97.861513) (width 0.25) (layer "F.Cu") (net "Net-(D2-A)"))
 (segment (start 104.385285 107.288889) (end 104.754102 105.912444) (width 0.25) (layer "F.Cu") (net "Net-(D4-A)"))
 (segment (start 112.5 101.525) (end 112.5 100.1) (width 0.25) (layer "F.Cu") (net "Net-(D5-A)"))
 (segment (start 85.375 93.4) (end 86.8 93.4) (width 0.25) (layer "F.Cu") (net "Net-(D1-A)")))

